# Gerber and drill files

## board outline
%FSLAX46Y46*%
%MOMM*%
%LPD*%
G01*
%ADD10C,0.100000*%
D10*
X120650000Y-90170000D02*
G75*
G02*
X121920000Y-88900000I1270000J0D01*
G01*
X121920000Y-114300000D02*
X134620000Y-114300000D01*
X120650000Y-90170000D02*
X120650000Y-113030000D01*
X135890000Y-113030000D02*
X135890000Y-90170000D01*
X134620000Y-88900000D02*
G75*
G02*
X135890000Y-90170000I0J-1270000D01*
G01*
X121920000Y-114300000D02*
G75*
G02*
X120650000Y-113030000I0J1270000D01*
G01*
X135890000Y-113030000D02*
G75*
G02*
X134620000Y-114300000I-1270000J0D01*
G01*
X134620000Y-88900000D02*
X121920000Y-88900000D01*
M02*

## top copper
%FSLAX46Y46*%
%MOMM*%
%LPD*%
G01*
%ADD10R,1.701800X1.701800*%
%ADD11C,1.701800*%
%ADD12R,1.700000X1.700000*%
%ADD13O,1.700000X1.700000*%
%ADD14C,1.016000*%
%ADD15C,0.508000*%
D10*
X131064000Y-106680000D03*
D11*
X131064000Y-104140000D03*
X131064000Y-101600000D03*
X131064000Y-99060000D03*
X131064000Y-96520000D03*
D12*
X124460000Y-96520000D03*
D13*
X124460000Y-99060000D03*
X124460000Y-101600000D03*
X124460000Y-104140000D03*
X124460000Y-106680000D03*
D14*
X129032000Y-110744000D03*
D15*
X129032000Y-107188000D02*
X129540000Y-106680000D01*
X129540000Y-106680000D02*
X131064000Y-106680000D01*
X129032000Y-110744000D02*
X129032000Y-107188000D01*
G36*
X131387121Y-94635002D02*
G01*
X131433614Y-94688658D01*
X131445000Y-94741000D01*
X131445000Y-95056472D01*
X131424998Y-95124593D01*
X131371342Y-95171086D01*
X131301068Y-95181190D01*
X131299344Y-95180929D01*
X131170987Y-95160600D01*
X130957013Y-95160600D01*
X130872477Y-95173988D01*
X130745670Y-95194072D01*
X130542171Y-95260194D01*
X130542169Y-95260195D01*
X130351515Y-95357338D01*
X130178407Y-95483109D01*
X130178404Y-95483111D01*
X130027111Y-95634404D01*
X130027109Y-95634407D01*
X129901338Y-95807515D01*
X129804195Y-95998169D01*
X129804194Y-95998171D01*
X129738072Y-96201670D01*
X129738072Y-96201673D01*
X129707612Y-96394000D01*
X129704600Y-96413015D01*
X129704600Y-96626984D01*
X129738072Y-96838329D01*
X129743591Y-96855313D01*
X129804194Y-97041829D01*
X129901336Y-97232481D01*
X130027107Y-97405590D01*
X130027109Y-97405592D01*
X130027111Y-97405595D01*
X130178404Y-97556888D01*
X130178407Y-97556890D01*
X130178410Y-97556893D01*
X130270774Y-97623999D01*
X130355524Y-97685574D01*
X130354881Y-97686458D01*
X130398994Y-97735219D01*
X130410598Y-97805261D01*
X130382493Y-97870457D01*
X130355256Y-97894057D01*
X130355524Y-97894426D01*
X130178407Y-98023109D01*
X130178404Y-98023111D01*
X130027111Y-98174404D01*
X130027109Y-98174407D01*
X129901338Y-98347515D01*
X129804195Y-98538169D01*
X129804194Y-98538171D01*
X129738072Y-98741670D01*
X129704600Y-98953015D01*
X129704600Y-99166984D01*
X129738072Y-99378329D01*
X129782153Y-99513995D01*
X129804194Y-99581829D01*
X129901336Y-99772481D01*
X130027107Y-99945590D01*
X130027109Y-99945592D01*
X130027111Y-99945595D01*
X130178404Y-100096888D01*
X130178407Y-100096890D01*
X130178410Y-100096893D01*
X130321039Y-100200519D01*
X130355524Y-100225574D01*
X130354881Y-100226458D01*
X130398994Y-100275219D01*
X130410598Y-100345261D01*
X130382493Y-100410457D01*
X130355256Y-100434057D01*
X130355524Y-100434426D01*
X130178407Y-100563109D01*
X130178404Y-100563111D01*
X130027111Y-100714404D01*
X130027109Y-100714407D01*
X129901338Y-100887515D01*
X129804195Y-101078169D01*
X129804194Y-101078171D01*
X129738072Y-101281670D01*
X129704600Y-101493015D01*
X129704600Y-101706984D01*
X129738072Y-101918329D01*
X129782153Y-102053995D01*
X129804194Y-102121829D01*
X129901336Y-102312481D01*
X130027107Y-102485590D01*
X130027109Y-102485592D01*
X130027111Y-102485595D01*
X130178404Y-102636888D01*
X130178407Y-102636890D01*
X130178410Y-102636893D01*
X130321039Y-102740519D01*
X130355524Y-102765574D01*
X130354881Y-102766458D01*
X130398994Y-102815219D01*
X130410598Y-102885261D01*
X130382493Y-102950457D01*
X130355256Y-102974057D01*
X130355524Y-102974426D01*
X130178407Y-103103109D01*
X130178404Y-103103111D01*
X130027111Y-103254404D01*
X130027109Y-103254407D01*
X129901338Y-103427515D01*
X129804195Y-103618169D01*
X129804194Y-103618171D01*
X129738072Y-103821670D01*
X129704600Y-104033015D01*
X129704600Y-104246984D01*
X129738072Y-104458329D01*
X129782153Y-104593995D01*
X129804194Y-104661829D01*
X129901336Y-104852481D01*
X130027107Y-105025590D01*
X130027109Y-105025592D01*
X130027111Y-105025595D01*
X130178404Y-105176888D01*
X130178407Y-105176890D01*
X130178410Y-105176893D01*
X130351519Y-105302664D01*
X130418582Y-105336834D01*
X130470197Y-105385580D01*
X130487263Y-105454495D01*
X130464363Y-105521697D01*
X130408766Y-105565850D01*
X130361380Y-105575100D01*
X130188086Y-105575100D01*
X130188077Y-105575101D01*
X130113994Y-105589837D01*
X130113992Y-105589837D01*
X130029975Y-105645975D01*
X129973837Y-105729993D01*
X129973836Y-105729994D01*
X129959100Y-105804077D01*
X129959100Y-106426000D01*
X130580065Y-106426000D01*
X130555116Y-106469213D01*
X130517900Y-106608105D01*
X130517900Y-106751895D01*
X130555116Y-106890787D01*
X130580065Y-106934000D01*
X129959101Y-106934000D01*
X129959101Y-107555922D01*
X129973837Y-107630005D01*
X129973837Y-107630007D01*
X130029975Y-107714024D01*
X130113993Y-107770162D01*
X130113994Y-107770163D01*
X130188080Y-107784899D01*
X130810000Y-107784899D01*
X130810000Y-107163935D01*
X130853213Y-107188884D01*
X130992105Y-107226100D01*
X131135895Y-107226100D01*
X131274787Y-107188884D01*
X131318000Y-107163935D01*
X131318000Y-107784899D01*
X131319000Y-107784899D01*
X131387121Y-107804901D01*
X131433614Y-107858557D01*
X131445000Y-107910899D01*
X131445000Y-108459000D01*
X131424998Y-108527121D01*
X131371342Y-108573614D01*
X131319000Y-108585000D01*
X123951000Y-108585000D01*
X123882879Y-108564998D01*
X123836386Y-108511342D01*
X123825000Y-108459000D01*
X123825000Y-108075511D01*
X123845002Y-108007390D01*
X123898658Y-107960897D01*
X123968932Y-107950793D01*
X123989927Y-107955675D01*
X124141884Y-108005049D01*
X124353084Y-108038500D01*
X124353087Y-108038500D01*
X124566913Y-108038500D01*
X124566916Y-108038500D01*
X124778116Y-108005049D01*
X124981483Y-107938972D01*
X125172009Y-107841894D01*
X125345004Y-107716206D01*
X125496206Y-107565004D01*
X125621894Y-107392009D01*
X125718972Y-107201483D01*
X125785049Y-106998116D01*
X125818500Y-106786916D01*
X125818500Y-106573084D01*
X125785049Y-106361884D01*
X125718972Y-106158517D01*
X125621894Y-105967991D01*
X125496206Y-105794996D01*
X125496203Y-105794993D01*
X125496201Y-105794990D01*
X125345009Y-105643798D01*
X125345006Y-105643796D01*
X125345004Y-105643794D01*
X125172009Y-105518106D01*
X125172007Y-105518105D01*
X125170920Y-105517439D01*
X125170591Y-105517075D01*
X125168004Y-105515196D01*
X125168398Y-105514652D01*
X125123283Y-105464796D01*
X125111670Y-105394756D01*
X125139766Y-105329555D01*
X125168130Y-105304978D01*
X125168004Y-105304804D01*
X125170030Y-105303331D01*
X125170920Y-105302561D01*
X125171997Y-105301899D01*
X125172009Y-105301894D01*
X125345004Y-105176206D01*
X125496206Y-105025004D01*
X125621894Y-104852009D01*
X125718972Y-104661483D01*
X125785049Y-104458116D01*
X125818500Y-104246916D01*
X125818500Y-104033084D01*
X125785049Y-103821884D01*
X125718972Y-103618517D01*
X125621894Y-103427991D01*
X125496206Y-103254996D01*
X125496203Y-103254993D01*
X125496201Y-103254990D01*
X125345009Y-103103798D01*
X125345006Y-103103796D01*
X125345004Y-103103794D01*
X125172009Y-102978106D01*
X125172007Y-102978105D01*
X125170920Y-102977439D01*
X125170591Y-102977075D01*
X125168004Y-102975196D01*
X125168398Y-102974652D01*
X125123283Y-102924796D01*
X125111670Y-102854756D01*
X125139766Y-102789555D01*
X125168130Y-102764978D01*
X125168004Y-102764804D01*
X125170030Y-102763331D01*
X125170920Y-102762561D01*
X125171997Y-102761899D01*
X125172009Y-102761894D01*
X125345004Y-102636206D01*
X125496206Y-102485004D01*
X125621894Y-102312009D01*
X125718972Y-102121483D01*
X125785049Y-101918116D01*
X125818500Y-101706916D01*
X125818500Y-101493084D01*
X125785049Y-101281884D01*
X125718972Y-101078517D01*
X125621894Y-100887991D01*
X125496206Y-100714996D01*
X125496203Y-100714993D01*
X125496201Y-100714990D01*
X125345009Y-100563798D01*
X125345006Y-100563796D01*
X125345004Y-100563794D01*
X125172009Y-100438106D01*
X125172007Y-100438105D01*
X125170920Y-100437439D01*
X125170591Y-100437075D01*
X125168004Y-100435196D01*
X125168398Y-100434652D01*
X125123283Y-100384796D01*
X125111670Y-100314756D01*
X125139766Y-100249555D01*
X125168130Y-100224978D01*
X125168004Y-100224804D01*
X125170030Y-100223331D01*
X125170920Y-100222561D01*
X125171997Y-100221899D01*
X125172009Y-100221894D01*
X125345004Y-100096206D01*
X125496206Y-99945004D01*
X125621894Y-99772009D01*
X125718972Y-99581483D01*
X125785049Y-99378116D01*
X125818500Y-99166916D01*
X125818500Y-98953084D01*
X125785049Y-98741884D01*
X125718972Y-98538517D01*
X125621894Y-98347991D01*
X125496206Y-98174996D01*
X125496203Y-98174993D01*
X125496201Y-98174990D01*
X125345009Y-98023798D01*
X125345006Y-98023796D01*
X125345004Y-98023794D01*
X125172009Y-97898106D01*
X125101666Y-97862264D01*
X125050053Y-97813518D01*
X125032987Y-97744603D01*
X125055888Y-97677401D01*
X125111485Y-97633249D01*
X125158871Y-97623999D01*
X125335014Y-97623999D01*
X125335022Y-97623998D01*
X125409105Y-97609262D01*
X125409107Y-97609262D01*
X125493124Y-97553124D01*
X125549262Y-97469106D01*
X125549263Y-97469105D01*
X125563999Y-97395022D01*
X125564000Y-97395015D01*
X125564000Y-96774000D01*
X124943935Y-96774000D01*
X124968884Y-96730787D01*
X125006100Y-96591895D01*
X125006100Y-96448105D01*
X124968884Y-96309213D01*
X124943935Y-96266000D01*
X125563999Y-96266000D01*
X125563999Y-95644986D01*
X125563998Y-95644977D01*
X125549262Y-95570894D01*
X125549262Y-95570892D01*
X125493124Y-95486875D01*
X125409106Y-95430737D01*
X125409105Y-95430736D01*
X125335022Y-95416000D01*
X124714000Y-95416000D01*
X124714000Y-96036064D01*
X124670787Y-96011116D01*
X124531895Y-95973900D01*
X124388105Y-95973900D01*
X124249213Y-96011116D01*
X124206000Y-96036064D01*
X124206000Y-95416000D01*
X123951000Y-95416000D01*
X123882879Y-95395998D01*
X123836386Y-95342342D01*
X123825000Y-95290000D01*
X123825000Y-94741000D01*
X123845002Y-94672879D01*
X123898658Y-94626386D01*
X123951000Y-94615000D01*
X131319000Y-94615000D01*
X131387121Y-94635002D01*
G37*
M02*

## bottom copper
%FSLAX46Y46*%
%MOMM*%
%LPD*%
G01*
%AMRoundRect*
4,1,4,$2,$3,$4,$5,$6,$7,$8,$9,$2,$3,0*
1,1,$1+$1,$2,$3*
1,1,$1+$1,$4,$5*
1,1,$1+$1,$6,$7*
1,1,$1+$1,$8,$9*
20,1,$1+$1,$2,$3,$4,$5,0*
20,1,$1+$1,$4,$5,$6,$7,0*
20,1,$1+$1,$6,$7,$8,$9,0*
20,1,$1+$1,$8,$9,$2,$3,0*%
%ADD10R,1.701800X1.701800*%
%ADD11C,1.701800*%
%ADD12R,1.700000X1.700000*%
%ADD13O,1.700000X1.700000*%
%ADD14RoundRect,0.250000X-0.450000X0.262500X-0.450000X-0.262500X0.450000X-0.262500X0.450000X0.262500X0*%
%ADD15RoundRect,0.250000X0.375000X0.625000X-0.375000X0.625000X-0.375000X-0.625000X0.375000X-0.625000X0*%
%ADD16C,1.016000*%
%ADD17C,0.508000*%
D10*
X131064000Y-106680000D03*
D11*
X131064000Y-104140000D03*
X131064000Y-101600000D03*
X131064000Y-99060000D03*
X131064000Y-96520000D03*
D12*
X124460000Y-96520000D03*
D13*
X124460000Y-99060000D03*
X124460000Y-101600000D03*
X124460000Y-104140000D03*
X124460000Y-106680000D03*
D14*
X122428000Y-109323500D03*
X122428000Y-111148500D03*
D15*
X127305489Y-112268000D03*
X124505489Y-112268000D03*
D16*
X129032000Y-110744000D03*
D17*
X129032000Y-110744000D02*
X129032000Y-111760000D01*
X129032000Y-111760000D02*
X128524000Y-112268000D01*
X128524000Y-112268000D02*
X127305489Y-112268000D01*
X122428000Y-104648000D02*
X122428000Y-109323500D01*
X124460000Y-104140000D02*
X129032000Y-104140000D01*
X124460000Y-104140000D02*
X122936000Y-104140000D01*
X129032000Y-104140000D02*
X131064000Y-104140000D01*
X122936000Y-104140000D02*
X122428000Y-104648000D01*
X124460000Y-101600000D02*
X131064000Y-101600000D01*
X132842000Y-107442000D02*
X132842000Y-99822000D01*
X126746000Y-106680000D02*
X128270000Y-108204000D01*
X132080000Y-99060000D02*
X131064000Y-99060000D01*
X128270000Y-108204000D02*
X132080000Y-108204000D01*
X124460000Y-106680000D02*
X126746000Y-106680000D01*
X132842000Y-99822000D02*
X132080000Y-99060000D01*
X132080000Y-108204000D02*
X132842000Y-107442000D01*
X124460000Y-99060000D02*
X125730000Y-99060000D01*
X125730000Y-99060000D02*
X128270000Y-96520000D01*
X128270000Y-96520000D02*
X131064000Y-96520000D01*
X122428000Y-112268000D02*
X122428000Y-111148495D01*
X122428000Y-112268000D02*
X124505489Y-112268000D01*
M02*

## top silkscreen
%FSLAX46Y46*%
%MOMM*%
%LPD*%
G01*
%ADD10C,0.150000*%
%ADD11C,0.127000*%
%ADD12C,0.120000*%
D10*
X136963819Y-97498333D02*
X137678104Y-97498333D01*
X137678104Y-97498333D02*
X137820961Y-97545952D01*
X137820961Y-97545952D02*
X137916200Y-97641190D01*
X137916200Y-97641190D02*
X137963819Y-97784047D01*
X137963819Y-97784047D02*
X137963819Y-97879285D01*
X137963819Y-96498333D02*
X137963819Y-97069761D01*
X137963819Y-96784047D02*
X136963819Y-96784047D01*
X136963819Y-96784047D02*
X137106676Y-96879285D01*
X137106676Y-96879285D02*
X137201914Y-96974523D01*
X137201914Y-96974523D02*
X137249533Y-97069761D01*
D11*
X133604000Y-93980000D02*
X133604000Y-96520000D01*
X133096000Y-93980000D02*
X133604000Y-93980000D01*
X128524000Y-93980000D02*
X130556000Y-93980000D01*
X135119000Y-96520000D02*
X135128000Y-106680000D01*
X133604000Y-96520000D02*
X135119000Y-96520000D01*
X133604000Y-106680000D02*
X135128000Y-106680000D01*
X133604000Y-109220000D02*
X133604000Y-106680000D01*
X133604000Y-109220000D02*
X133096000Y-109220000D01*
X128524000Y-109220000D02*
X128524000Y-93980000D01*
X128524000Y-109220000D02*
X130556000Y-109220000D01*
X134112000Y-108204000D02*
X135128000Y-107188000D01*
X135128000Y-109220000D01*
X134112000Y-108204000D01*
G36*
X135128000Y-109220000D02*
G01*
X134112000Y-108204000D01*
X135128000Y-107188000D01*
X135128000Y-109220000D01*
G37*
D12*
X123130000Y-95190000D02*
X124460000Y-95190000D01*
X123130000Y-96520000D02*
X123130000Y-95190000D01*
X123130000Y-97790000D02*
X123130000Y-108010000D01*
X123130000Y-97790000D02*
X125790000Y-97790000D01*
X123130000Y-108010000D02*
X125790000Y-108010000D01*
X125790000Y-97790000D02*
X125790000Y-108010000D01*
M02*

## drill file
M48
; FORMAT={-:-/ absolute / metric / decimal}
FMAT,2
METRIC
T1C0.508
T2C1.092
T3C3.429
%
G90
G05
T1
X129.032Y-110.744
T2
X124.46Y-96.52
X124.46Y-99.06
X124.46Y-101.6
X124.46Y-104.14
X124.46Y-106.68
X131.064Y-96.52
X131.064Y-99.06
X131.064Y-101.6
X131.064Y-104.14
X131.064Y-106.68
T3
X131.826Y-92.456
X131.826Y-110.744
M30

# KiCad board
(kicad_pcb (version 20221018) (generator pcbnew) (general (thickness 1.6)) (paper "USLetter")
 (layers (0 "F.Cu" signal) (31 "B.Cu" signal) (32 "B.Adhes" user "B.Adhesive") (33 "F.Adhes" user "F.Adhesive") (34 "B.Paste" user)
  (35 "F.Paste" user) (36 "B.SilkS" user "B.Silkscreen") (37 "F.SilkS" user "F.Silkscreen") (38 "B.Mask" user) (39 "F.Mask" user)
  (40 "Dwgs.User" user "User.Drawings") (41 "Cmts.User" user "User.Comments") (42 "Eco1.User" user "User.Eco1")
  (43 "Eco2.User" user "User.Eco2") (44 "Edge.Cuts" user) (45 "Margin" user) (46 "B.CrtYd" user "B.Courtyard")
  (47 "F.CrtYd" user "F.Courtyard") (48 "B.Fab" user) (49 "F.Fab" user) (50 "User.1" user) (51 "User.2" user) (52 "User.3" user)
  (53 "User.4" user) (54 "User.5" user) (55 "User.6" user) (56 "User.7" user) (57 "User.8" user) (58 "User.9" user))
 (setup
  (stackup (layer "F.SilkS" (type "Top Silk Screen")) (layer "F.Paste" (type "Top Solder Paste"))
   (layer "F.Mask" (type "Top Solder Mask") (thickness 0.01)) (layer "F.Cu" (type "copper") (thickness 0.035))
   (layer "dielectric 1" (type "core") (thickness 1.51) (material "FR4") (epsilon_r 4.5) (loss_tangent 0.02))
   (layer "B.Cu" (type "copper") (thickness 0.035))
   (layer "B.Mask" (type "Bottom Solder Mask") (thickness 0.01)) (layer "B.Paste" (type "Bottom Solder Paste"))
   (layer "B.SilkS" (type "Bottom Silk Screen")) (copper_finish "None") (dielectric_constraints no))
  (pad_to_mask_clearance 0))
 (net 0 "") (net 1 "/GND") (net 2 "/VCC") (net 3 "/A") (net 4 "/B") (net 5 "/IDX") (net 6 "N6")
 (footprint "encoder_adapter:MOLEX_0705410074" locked (layer "F.Cu") (at 131.064 106.68 -90)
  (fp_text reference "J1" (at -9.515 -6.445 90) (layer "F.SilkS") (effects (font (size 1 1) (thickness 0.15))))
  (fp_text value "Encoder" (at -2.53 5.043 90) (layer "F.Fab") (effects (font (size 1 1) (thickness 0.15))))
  (fp_line (start -12.7 -2.54) (end -10.16 -2.54) (stroke (width 0.127) (type solid)) (layer "F.SilkS"))
  (fp_line (start -12.7 -2.032) (end -12.7 -2.54) (stroke (width 0.127) (type solid)) (layer "F.SilkS"))
  (fp_line (start -12.7 2.54) (end -12.7 0.508) (stroke (width 0.127) (type solid)) (layer "F.SilkS"))
  (fp_line (start -10.16 -4.055) (end 0 -4.064) (stroke (width 0.127) (type solid)) (layer "F.SilkS"))
  (fp_line (start -10.16 -2.54) (end -10.16 -4.055) (stroke (width 0.127) (type solid)) (layer "F.SilkS"))
  (fp_line (start 0 -2.54) (end 0 -4.064) (stroke (width 0.127) (type solid)) (layer "F.SilkS"))
  (fp_line (start 2.54 -2.54) (end 0 -2.54) (stroke (width 0.127) (type solid)) (layer "F.SilkS"))
  (fp_line (start 2.54 -2.54) (end 2.54 -2.032) (stroke (width 0.127) (type solid)) (layer "F.SilkS"))
  (fp_line (start 2.54 2.54) (end -12.7 2.54) (stroke (width 0.127) (type solid)) (layer "F.SilkS"))
  (fp_line (start 2.54 2.54) (end 2.54 0.508) (stroke (width 0.127) (type solid)) (layer "F.SilkS"))
  (fp_poly (pts (xy 1.524 -3.048) (xy 0.508 -4.064) (xy 2.54 -4.064)) (stroke (width 0.127) (type solid)) (fill solid) (layer "F.SilkS"))
  (pad "" np_thru_hole circle locked (at -14.224 -0.762 270) (size 1.524 1.524) (drill 3.429) (layers "F&B.Cu" "*.Mask"))
  (pad "" np_thru_hole circle locked (at 4.064 -0.762 270) (size 1.524 1.524) (drill 3.429) (layers "F&B.Cu" "*.Mask"))
  (pad "1" thru_hole rect locked (at 0 0 270) (size 1.7018 1.7018) (drill 1.0922) (layers "*.Cu") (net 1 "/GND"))
  (pad "2" thru_hole circle locked (at -2.54 0 270) (size 1.7018 1.7018) (drill 1.0922) (layers "*.Cu") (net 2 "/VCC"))
  (pad "3" thru_hole circle locked (at -5.08 0 270) (size 1.7018 1.7018) (drill 1.0922) (layers "*.Cu") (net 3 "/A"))
  (pad "4" thru_hole circle locked (at -7.62 0 270) (size 1.7018 1.7018) (drill 1.0922) (layers "*.Cu") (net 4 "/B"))
  (pad "5" thru_hole circle locked (at -10.16 0 270) (size 1.7018 1.7018) (drill 1.0922) (layers "*.Cu") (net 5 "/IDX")))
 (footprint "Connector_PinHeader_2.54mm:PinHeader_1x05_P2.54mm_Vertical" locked (layer "F.Cu") (at 124.46 96.52)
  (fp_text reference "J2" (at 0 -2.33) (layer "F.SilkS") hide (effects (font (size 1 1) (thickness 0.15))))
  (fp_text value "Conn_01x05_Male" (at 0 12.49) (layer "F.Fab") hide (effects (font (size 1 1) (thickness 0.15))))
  (fp_line (start -1.33 -1.33) (end 0 -1.33) (stroke (width 0.12) (type solid)) (layer "F.SilkS"))
  (fp_line (start -1.33 0) (end -1.33 -1.33) (stroke (width 0.12) (type solid)) (layer "F.SilkS"))
  (fp_line (start -1.33 1.27) (end -1.33 11.49) (stroke (width 0.12) (type solid)) (layer "F.SilkS"))
  (fp_line (start -1.33 1.27) (end 1.33 1.27) (stroke (width 0.12) (type solid)) (layer "F.SilkS"))
  (fp_line (start -1.33 11.49) (end 1.33 11.49) (stroke (width 0.12) (type solid)) (layer "F.SilkS"))
  (fp_line (start 1.33 1.27) (end 1.33 11.49) (stroke (width 0.12) (type solid)) (layer "F.SilkS"))
  (pad "1" thru_hole rect locked (at 0 0) (size 1.7 1.7) (drill 1.0922) (layers "*.Cu" "*.Mask") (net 1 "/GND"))
  (pad "2" thru_hole oval locked (at 0 2.54) (size 1.7 1.7) (drill 1.0922) (layers "*.Cu" "*.Mask") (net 5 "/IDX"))
  (pad "3" thru_hole oval locked (at 0 5.08) (size 1.7 1.7) (drill 1.0922) (layers "*.Cu" "*.Mask") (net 3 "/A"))
  (pad "4" thru_hole oval locked (at 0 7.62) (size 1.7 1.7) (drill 1.0922) (layers "*.Cu" "*.Mask") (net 2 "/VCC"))
  (pad "5" thru_hole oval locked (at 0 10.16) (size 1.7 1.7) (drill 1.0922) (layers "*.Cu" "*.Mask") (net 4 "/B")))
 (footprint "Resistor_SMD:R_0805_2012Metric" (layer "B.Cu") (at 122.428 110.236 -90)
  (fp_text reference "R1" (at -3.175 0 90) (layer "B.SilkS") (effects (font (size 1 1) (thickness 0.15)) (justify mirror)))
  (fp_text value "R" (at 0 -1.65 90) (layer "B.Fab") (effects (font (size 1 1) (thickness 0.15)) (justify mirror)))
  (pad "1" smd roundrect (at -0.9125 0 270) (size 1.025 1.4) (layers "B.Cu" "B.Paste" "B.Mask") (roundrect_rratio 0.243902) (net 2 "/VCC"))
  (pad "2" smd roundrect (at 0.9125 0 270) (size 1.025 1.4) (layers "B.Cu" "B.Paste" "B.Mask") (roundrect_rratio 0.243902) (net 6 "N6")))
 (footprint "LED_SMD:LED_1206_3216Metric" (layer "B.Cu") (at 125.905489 112.268 180)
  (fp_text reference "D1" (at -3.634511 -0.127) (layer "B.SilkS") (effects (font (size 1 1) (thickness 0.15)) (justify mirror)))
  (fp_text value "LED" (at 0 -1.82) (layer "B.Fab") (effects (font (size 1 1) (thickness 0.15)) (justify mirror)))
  (pad "1" smd roundrect (at -1.4 0 180) (size 1.25 1.75) (layers "B.Cu" "B.Paste" "B.Mask") (roundrect_rratio 0.2) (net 1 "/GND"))
  (pad "2" smd roundrect (at 1.4 0 180) (size 1.25 1.75) (layers "B.Cu" "B.Paste" "B.Mask") (roundrect_rratio 0.2) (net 6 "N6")))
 (gr_arc (start 120.65 90.17) (mid 121.021974 89.271974) (end 121.92 88.9) (stroke (width 0.1) (type solid)) (layer "Edge.Cuts"))
 (gr_line (start 121.92 114.3) (end 134.62 114.3) (stroke (width 0.1) (type solid)) (layer "Edge.Cuts"))
 (gr_line (start 120.65 90.17) (end 120.65 113.03) (stroke (width 0.1) (type solid)) (layer "Edge.Cuts"))
 (gr_line (start 135.89 113.03) (end 135.89 90.17) (stroke (width 0.1) (type solid)) (layer "Edge.Cuts"))
 (gr_arc (start 134.62 88.9) (mid 135.518026 89.271974) (end 135.89 90.17) (stroke (width 0.1) (type solid)) (layer "Edge.Cuts"))
 (gr_arc (start 121.92 114.3) (mid 121.021974 113.928026) (end 120.65 113.03) (stroke (width 0.1) (type solid)) (layer "Edge.Cuts"))
 (gr_arc (start 135.89 113.03) (mid 135.518026 113.928026) (end 134.62 114.3) (stroke (width 0.1) (type solid)) (layer "Edge.Cuts"))
 (gr_line (start 134.62 88.9) (end 121.92 88.9) (stroke (width 0.1) (type solid)) (layer "Edge.Cuts"))
 (segment (start 129.032 107.188) (end 129.54 106.68) (width 0.508) (layer "F.Cu") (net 1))
 (segment (start 129.54 106.68) (end 131.064 106.68) (width 0.508) (layer "F.Cu") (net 1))
 (segment (start 129.032 110.744) (end 129.032 107.188) (width 0.508) (layer "F.Cu") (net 1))
 (via (at 129.032 110.744) (size 1.016) (drill 0.508) (layers "F.Cu" "B.Cu") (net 1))
 (segment (start 129.032 110.744) (end 129.032 111.76) (width 0.508) (layer "B.Cu") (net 1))
 (segment (start 129.032 111.76) (end 128.524 112.268) (width 0.508) (layer "B.Cu") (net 1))
 (segment (start 128.524 112.268) (end 127.305489 112.268) (width 0.508) (layer "B.Cu") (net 1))
 (segment (start 122.428 104.648) (end 122.428 109.3235) (width 0.508) (layer "B.Cu") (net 2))
 (segment (start 124.46 104.14) (end 129.032 104.14) (width 0.508) (layer "B.Cu") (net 2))
 (segment (start 124.46 104.14) (end 122.936 104.14) (width 0.508) (layer "B.Cu") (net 2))
 (segment (start 129.032 104.14) (end 131.064 104.14) (width 0.508) (layer "B.Cu") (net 2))
 (segment (start 122.936 104.14) (end 122.428 104.648) (width 0.508) (layer "B.Cu") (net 2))
 (segment (start 124.46 101.6) (end 131.064 101.6) (width 0.508) (layer "B.Cu") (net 3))
 (segment (start 132.842 107.442) (end 132.842 99.822) (width 0.508) (layer "B.Cu") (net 4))
 (segment (start 126.746 106.68) (end 128.27 108.204) (width 0.508) (layer "B.Cu") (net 4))
 (segment (start 132.08 99.06) (end 131.064 99.06) (width 0.508) (layer "B.Cu") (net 4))
 (segment (start 128.27 108.204) (end 132.08 108.204) (width 0.508) (layer "B.Cu") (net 4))
 (segment (start 124.46 106.68) (end 126.746 106.68) (width 0.508) (layer "B.Cu") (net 4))
 (segment (start 132.842 99.822) (end 132.08 99.06) (width 0.508) (layer "B.Cu") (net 4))
 (segment (start 132.08 108.204) (end 132.842 107.442) (width 0.508) (layer "B.Cu") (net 4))
 (segment (start 124.46 99.06) (end 125.73 99.06) (width 0.508) (layer "B.Cu") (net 5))
 (segment (start 125.73 99.06) (end 128.27 96.52) (width 0.508) (layer "B.Cu") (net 5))
 (segment (start 128.27 96.52) (end 131.064 96.52) (width 0.508) (layer "B.Cu") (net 5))
 (segment (start 122.428 112.268) (end 122.428 111.148495) (width 0.508) (layer "B.Cu") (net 6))
 (segment (start 122.428 112.268) (end 124.505489 112.268) (width 0.508) (layer "B.Cu") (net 6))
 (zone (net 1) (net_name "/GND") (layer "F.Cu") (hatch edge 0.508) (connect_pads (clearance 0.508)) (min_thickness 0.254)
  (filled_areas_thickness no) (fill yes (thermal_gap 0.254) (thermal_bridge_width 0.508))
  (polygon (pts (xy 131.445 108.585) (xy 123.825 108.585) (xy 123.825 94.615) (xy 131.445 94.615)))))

